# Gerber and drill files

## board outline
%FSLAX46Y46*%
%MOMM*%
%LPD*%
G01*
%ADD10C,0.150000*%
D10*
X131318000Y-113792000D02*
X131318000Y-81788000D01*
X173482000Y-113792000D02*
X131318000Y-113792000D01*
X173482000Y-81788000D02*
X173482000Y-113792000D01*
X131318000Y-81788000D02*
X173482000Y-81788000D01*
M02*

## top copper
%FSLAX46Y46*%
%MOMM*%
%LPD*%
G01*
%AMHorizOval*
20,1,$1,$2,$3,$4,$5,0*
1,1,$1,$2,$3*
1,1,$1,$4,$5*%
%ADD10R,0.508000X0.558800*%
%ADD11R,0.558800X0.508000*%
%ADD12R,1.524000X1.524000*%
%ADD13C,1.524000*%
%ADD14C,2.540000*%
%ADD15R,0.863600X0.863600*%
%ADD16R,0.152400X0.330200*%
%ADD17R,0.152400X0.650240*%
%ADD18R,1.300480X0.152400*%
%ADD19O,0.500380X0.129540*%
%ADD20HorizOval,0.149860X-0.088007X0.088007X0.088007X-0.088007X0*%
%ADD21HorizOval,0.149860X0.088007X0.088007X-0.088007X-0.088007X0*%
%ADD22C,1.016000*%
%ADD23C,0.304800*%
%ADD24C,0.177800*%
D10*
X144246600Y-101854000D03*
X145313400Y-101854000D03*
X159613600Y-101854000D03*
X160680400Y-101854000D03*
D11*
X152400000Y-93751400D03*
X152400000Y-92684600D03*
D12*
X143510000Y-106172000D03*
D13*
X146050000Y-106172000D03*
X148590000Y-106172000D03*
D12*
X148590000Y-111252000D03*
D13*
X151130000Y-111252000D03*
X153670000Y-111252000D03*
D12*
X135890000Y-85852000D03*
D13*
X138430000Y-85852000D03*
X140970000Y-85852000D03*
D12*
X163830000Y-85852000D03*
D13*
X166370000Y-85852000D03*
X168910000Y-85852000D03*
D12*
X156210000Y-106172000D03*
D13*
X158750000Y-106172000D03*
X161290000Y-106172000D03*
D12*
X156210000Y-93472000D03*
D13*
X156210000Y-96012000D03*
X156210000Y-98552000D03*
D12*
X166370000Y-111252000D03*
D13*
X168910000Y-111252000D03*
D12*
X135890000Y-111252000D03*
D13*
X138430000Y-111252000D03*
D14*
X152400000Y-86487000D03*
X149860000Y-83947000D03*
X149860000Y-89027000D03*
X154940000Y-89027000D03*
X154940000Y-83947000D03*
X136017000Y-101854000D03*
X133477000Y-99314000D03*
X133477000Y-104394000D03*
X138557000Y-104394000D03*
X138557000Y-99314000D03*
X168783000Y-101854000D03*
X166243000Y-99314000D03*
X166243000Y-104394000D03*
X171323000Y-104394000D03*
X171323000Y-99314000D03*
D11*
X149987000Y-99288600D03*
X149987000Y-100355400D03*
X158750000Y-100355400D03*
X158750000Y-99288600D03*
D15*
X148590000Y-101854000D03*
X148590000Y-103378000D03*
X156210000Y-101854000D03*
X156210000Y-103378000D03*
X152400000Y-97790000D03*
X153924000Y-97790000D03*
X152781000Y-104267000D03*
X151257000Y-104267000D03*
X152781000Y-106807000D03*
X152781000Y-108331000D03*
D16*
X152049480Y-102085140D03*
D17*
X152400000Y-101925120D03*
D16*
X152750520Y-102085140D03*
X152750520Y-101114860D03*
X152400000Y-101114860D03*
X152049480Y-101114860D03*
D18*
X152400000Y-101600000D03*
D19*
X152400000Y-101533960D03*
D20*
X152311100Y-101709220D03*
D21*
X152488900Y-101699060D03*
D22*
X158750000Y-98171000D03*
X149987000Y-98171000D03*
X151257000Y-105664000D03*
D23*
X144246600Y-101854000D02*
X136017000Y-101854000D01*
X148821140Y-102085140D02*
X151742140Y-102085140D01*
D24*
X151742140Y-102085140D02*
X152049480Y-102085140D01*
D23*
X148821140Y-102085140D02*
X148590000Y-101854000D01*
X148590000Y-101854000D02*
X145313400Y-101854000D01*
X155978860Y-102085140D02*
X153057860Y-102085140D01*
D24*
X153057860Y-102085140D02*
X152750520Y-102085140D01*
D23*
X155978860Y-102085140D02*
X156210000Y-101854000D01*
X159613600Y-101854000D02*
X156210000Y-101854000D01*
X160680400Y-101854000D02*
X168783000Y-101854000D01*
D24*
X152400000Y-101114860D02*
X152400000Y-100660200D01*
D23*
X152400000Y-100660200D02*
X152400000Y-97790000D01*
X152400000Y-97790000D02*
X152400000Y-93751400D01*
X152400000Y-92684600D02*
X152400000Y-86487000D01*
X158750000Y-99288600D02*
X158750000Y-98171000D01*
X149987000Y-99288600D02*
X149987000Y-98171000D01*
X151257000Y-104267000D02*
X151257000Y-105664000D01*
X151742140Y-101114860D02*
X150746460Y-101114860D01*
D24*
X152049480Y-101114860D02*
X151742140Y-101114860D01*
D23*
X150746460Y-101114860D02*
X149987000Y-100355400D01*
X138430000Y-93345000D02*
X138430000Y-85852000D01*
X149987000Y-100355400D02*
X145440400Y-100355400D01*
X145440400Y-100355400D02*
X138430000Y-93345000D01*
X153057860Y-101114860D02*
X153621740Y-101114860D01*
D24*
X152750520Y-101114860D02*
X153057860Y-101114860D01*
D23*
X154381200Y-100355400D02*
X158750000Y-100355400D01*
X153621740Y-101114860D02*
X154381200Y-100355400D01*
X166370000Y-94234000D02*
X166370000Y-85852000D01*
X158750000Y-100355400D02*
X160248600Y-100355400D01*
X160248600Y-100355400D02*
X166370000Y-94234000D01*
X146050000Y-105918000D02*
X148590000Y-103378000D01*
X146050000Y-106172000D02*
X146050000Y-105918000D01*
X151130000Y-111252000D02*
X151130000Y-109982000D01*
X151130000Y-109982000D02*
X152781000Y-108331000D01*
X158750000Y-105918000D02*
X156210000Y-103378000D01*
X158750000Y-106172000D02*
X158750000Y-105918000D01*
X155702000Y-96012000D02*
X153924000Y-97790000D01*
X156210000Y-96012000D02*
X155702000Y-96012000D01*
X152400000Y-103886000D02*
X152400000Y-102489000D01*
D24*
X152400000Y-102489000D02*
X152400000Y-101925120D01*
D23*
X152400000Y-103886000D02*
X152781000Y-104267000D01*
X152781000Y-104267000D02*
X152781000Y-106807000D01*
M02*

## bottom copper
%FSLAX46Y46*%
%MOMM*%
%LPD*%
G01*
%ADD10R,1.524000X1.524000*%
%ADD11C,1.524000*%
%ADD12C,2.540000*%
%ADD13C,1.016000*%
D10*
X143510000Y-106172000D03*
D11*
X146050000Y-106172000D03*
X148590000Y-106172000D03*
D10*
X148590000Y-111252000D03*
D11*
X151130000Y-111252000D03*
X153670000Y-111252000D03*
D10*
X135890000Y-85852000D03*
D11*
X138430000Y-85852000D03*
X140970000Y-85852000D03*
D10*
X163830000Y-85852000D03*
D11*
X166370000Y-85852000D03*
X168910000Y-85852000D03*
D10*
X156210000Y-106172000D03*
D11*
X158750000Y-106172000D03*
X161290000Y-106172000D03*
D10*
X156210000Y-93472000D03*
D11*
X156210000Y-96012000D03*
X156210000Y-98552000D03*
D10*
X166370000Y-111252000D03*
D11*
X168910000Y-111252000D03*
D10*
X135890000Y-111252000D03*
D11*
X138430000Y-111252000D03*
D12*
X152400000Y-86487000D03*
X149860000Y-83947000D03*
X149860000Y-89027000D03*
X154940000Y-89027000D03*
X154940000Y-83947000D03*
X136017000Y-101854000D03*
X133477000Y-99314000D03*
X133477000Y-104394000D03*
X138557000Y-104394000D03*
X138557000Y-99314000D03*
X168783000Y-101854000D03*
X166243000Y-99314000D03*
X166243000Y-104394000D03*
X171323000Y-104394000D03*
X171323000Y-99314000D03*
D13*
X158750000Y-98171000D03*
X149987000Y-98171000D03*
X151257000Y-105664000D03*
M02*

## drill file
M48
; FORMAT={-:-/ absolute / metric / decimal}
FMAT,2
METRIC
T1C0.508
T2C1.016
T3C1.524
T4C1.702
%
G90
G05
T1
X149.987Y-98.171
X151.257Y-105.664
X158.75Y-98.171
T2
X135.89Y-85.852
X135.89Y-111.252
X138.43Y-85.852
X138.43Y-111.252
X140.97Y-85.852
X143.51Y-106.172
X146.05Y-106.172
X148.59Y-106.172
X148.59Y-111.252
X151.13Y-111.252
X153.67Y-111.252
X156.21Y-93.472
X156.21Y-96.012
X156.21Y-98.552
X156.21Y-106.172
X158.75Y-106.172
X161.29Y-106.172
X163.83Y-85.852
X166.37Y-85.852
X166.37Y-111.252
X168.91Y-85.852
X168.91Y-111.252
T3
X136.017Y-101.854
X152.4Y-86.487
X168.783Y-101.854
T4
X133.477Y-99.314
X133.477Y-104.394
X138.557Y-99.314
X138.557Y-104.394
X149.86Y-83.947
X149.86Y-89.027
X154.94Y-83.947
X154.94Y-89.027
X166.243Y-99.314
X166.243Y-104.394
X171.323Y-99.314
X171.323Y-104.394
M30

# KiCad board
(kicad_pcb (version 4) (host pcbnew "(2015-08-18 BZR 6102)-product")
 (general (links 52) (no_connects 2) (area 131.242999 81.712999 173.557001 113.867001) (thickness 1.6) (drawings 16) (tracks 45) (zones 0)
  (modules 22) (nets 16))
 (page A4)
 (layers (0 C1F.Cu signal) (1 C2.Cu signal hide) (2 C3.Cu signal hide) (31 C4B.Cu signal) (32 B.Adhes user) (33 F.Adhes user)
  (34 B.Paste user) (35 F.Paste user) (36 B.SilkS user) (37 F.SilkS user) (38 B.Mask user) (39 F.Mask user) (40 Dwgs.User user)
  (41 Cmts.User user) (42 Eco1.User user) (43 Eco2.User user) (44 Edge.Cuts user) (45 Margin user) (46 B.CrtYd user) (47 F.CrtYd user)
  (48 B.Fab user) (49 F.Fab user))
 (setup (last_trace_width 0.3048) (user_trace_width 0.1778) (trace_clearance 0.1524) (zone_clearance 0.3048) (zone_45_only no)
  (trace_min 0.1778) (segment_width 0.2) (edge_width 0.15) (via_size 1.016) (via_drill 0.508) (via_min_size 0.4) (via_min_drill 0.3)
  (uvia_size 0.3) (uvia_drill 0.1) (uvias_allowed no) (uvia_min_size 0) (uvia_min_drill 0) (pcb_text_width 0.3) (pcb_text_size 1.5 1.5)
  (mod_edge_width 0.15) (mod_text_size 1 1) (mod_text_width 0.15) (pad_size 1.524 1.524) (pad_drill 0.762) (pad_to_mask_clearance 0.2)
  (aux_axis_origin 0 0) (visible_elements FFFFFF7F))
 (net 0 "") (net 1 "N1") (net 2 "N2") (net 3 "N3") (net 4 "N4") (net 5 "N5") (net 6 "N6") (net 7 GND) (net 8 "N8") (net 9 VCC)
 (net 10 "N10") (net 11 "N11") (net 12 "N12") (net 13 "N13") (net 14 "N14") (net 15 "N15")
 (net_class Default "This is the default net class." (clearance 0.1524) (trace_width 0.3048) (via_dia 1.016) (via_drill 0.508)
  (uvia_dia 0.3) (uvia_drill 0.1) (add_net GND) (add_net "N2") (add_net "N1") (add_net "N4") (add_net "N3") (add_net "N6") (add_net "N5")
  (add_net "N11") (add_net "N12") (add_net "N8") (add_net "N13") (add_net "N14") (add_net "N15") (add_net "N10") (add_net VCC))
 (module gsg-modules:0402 (layer C1F.Cu) (at 144.78 101.854 180) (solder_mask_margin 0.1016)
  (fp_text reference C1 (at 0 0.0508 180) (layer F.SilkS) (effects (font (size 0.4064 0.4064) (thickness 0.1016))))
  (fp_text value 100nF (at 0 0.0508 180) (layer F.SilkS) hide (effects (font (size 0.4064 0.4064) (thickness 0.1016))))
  (pad 2 smd rect (at 0.5334 0 180) (size 0.508 0.5588) (layers C1F.Cu F.Paste F.Mask) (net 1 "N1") (solder_mask_margin 0.1016))
  (pad 1 smd rect (at -0.5334 0 180) (size 0.508 0.5588) (layers C1F.Cu F.Paste F.Mask) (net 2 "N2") (solder_mask_margin 0.1016)))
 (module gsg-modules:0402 (layer C1F.Cu) (at 160.147 101.854 180) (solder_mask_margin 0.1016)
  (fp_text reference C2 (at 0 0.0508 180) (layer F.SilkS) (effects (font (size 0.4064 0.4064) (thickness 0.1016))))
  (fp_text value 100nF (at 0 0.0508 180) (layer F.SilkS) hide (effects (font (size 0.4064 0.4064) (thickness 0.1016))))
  (pad 2 smd rect (at 0.5334 0 180) (size 0.508 0.5588) (layers C1F.Cu F.Paste F.Mask) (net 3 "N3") (solder_mask_margin 0.1016))
  (pad 1 smd rect (at -0.5334 0 180) (size 0.508 0.5588) (layers C1F.Cu F.Paste F.Mask) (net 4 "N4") (solder_mask_margin 0.1016)))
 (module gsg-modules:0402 (layer C1F.Cu) (at 152.4 93.218 270) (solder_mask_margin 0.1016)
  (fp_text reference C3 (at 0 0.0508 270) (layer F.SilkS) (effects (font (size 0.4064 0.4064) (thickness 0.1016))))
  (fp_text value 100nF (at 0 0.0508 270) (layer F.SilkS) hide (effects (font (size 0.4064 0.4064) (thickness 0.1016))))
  (pad 2 smd rect (at 0.5334 0 270) (size 0.508 0.5588) (layers C1F.Cu F.Paste F.Mask) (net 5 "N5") (solder_mask_margin 0.1016))
  (pad 1 smd rect (at -0.5334 0 270) (size 0.508 0.5588) (layers C1F.Cu F.Paste F.Mask) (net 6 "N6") (solder_mask_margin 0.1016)))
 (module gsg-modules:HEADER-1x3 (layer C1F.Cu) (at 146.05 106.172)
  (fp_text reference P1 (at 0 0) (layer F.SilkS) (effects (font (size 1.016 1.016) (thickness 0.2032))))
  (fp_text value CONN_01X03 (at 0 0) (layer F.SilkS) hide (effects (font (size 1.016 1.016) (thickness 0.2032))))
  (pad 1 thru_hole rect (at -2.54 0) (size 1.524 1.524) (drill 1.016) (layers *.Cu *.Mask F.SilkS) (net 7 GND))
  (pad 2 thru_hole circle (at 0 0) (size 1.524 1.524) (drill 1.016) (layers *.Cu *.Mask F.SilkS) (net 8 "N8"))
  (pad 3 thru_hole circle (at 2.54 0) (size 1.524 1.524) (drill 1.016) (layers *.Cu *.Mask F.SilkS) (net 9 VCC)))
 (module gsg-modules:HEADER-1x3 (layer C1F.Cu) (at 151.13 111.252)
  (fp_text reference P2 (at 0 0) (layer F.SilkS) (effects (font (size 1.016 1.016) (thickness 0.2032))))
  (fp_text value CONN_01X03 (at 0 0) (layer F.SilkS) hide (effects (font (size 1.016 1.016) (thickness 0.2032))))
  (pad 1 thru_hole rect (at -2.54 0) (size 1.524 1.524) (drill 1.016) (layers *.Cu *.Mask F.SilkS) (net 7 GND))
  (pad 2 thru_hole circle (at 0 0) (size 1.524 1.524) (drill 1.016) (layers *.Cu *.Mask F.SilkS) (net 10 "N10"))
  (pad 3 thru_hole circle (at 2.54 0) (size 1.524 1.524) (drill 1.016) (layers *.Cu *.Mask F.SilkS) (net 9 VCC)))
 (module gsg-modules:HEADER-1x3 (layer C1F.Cu) (at 138.43 85.852)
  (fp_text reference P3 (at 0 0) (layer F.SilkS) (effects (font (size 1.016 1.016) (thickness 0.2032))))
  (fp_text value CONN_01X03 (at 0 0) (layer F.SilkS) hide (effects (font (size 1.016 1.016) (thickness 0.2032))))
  (pad 1 thru_hole rect (at -2.54 0) (size 1.524 1.524) (drill 1.016) (layers *.Cu *.Mask F.SilkS) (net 7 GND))
  (pad 2 thru_hole circle (at 0 0) (size 1.524 1.524) (drill 1.016) (layers *.Cu *.Mask F.SilkS) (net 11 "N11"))
  (pad 3 thru_hole circle (at 2.54 0) (size 1.524 1.524) (drill 1.016) (layers *.Cu *.Mask F.SilkS) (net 9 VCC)))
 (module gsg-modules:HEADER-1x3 (layer C1F.Cu) (at 166.37 85.852)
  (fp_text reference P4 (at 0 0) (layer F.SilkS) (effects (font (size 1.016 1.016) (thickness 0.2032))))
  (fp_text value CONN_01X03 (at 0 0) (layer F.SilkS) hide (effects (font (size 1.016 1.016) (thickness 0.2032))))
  (pad 1 thru_hole rect (at -2.54 0) (size 1.524 1.524) (drill 1.016) (layers *.Cu *.Mask F.SilkS) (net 7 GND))
  (pad 2 thru_hole circle (at 0 0) (size 1.524 1.524) (drill 1.016) (layers *.Cu *.Mask F.SilkS) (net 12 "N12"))
  (pad 3 thru_hole circle (at 2.54 0) (size 1.524 1.524) (drill 1.016) (layers *.Cu *.Mask F.SilkS) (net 9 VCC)))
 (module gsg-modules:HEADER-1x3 (layer C1F.Cu) (at 158.75 106.172)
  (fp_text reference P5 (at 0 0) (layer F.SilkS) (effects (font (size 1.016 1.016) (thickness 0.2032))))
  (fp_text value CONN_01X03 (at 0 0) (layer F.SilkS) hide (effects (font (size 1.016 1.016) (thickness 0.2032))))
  (pad 1 thru_hole rect (at -2.54 0) (size 1.524 1.524) (drill 1.016) (layers *.Cu *.Mask F.SilkS) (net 7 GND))
  (pad 2 thru_hole circle (at 0 0) (size 1.524 1.524) (drill 1.016) (layers *.Cu *.Mask F.SilkS) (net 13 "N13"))
  (pad 3 thru_hole circle (at 2.54 0) (size 1.524 1.524) (drill 1.016) (layers *.Cu *.Mask F.SilkS) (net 9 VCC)))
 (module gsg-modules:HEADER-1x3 (layer C1F.Cu) (at 156.21 96.012 270)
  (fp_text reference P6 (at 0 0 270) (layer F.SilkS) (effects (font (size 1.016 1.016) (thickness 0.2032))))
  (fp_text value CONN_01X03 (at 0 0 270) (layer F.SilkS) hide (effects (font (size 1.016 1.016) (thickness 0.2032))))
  (pad 1 thru_hole rect (at -2.54 0 270) (size 1.524 1.524) (drill 1.016) (layers *.Cu *.Mask F.SilkS) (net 7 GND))
  (pad 2 thru_hole circle (at 0 0 270) (size 1.524 1.524) (drill 1.016) (layers *.Cu *.Mask F.SilkS) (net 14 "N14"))
  (pad 3 thru_hole circle (at 2.54 0 270) (size 1.524 1.524) (drill 1.016) (layers *.Cu *.Mask F.SilkS) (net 9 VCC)))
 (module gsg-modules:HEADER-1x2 (layer C1F.Cu) (at 167.64 111.252)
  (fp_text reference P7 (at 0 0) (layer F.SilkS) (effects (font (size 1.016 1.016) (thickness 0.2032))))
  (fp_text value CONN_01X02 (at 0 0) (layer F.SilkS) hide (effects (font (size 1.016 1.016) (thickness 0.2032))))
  (pad 1 thru_hole rect (at -1.27 0) (size 1.524 1.524) (drill 1.016) (layers *.Cu *.Mask F.SilkS) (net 9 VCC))
  (pad 2 thru_hole circle (at 1.27 0) (size 1.524 1.524) (drill 1.016) (layers *.Cu *.Mask F.SilkS) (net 9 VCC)))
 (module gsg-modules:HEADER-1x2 (layer C1F.Cu) (at 137.16 111.252)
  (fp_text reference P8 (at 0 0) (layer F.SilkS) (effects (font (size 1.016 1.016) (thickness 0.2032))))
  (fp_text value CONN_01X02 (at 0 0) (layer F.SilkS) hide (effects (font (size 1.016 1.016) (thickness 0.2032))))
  (pad 1 thru_hole rect (at -1.27 0) (size 1.524 1.524) (drill 1.016) (layers *.Cu *.Mask F.SilkS) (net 7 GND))
  (pad 2 thru_hole circle (at 1.27 0) (size 1.524 1.524) (drill 1.016) (layers *.Cu *.Mask F.SilkS) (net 7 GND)))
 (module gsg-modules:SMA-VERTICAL (layer C1F.Cu) (at 152.4 86.487)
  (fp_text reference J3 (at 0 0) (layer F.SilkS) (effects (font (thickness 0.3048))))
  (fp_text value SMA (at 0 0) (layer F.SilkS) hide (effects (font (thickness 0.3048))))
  (pad 1 thru_hole circle (at 0 0) (size 2.54 2.54) (drill 1.524) (layers *.Cu *.Mask F.SilkS) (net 6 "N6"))
  (pad 2 thru_hole circle (at -2.54 -2.54) (size 2.54 2.54) (drill 1.7018) (layers *.Cu *.Mask F.SilkS) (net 7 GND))
  (pad 2 thru_hole circle (at -2.54 2.54) (size 2.54 2.54) (drill 1.7018) (layers *.Cu *.Mask F.SilkS) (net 7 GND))
  (pad 2 thru_hole circle (at 2.54 2.54) (size 2.54 2.54) (drill 1.7018) (layers *.Cu *.Mask F.SilkS) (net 7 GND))
  (pad 2 thru_hole circle (at 2.54 -2.54) (size 2.54 2.54) (drill 1.7018) (layers *.Cu *.Mask F.SilkS) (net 7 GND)))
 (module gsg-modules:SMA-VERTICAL (layer C1F.Cu) (at 136.017 101.854)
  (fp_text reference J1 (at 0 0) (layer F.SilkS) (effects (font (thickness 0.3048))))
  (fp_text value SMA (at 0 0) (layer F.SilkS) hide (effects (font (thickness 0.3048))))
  (pad 1 thru_hole circle (at 0 0) (size 2.54 2.54) (drill 1.524) (layers *.Cu *.Mask F.SilkS) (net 1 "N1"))
  (pad 2 thru_hole circle (at -2.54 -2.54) (size 2.54 2.54) (drill 1.7018) (layers *.Cu *.Mask F.SilkS) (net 7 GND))
  (pad 2 thru_hole circle (at -2.54 2.54) (size 2.54 2.54) (drill 1.7018) (layers *.Cu *.Mask F.SilkS) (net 7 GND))
  (pad 2 thru_hole circle (at 2.54 2.54) (size 2.54 2.54) (drill 1.7018) (layers *.Cu *.Mask F.SilkS) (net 7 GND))
  (pad 2 thru_hole circle (at 2.54 -2.54) (size 2.54 2.54) (drill 1.7018) (layers *.Cu *.Mask F.SilkS) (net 7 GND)))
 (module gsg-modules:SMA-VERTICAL (layer C1F.Cu) (at 168.783 101.854)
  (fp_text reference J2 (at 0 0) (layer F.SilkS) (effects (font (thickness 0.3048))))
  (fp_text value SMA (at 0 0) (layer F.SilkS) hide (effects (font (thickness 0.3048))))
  (pad 1 thru_hole circle (at 0 0) (size 2.54 2.54) (drill 1.524) (layers *.Cu *.Mask F.SilkS) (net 4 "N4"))
  (pad 2 thru_hole circle (at -2.54 -2.54) (size 2.54 2.54) (drill 1.7018) (layers *.Cu *.Mask F.SilkS) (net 7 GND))
  (pad 2 thru_hole circle (at -2.54 2.54) (size 2.54 2.54) (drill 1.7018) (layers *.Cu *.Mask F.SilkS) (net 7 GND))
  (pad 2 thru_hole circle (at 2.54 2.54) (size 2.54 2.54) (drill 1.7018) (layers *.Cu *.Mask F.SilkS) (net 7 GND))
  (pad 2 thru_hole circle (at 2.54 -2.54) (size 2.54 2.54) (drill 1.7018) (layers *.Cu *.Mask F.SilkS) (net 7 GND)))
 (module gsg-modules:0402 (layer C1F.Cu) (at 149.987 99.822 90) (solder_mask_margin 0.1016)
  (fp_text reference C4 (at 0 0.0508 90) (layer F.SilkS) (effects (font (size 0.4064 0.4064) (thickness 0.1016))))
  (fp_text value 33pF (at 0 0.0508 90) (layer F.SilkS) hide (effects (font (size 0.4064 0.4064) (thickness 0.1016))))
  (pad 2 smd rect (at 0.5334 0 90) (size 0.508 0.5588) (layers C1F.Cu F.Paste F.Mask) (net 7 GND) (solder_mask_margin 0.1016))
  (pad 1 smd rect (at -0.5334 0 90) (size 0.508 0.5588) (layers C1F.Cu F.Paste F.Mask) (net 11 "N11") (solder_mask_margin 0.1016)))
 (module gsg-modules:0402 (layer C1F.Cu) (at 158.75 99.822 270) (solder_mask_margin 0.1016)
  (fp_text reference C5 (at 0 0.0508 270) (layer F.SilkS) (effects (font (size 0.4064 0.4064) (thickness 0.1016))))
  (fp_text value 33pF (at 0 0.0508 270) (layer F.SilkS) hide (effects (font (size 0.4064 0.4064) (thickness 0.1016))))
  (pad 2 smd rect (at 0.5334 0 270) (size 0.508 0.5588) (layers C1F.Cu F.Paste F.Mask) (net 12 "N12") (solder_mask_margin 0.1016))
  (pad 1 smd rect (at -0.5334 0 270) (size 0.508 0.5588) (layers C1F.Cu F.Paste F.Mask) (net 7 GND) (solder_mask_margin 0.1016)))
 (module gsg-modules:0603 (layer C1F.Cu) (at 148.59 102.616 90) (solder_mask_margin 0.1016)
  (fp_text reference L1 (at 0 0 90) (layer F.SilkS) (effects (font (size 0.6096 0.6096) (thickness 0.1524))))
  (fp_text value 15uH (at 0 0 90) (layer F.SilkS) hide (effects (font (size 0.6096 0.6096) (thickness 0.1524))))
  (pad 2 smd rect (at 0.762 0 90) (size 0.8636 0.8636) (layers C1F.Cu F.Paste F.Mask) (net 2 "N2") (solder_mask_margin 0.1016)
   (clearance 0.1778))
  (pad 1 smd rect (at -0.762 0 90) (size 0.8636 0.8636) (layers C1F.Cu F.Paste F.Mask) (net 8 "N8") (solder_mask_margin 0.1016)
   (clearance 0.1778)))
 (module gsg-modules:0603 (layer C1F.Cu) (at 156.21 102.616 90) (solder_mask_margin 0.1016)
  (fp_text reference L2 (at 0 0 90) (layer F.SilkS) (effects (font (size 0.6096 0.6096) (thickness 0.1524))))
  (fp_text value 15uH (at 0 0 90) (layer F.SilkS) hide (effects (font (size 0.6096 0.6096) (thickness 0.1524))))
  (pad 2 smd rect (at 0.762 0 90) (size 0.8636 0.8636) (layers C1F.Cu F.Paste F.Mask) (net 3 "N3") (solder_mask_margin 0.1016)
   (clearance 0.1778))
  (pad 1 smd rect (at -0.762 0 90) (size 0.8636 0.8636) (layers C1F.Cu F.Paste F.Mask) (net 13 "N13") (solder_mask_margin 0.1016)
   (clearance 0.1778)))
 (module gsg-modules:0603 (layer C1F.Cu) (at 153.162 97.79 180) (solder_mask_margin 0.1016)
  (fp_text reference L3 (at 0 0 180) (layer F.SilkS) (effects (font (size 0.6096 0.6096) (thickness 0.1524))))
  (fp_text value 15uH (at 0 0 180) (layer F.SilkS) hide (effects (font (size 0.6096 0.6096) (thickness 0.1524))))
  (pad 2 smd rect (at 0.762 0 180) (size 0.8636 0.8636) (layers C1F.Cu F.Paste F.Mask) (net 5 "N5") (solder_mask_margin 0.1016)
   (clearance 0.1778))
  (pad 1 smd rect (at -0.762 0 180) (size 0.8636 0.8636) (layers C1F.Cu F.Paste F.Mask) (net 14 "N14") (solder_mask_margin 0.1016)
   (clearance 0.1778)))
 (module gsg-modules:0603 (layer C1F.Cu) (at 152.019 104.267) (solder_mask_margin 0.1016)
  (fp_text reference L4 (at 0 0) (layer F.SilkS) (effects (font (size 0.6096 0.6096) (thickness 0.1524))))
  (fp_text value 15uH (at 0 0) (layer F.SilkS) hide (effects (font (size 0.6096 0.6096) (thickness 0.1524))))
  (pad 2 smd rect (at 0.762 0) (size 0.8636 0.8636) (layers C1F.Cu F.Paste F.Mask) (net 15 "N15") (solder_mask_margin 0.1016)
   (clearance 0.1778))
  (pad 1 smd rect (at -0.762 0) (size 0.8636 0.8636) (layers C1F.Cu F.Paste F.Mask) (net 7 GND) (solder_mask_margin 0.1016)
   (clearance 0.1778)))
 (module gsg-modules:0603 (layer C1F.Cu) (at 152.781 107.569 90) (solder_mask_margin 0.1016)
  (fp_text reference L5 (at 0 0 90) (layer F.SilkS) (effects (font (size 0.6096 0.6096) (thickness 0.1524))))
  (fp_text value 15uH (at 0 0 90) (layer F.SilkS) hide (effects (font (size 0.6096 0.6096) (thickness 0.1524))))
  (pad 2 smd rect (at 0.762 0 90) (size 0.8636 0.8636) (layers C1F.Cu F.Paste F.Mask) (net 15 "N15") (solder_mask_margin 0.1016)
   (clearance 0.1778))
  (pad 1 smd rect (at -0.762 0 90) (size 0.8636 0.8636) (layers C1F.Cu F.Paste F.Mask) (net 10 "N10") (solder_mask_margin 0.1016)
   (clearance 0.1778)))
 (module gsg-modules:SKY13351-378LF (layer C1F.Cu) (at 152.4 101.6 90) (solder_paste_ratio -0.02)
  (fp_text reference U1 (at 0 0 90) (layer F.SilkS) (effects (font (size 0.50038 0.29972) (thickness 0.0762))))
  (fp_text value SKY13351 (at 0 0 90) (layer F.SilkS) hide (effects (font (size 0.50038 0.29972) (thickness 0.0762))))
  (pad 1 smd rect (at -0.48514 -0.35052 90) (size 0.3302 0.1524) (layers C1F.Cu F.Paste F.Mask) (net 2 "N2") (die_length -2147.483648))
  (pad 2 smd rect (at -0.32512 0 90) (size 0.65024 0.1524) (layers C1F.Cu F.Paste F.Mask) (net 15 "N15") (die_length -2147.483648))
  (pad 3 smd rect (at -0.48514 0.35052 90) (size 0.3302 0.1524) (layers C1F.Cu F.Paste F.Mask) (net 3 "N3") (die_length -2147.483648))
  (pad 4 smd rect (at 0.48514 0.35052 90) (size 0.3302 0.1524) (layers C1F.Cu F.Paste F.Mask) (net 12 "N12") (die_length 0.0508))
  (pad 5 smd rect (at 0.48514 0 90) (size 0.3302 0.1524) (layers C1F.Cu F.Paste F.Mask) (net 5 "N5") (die_length 10.53846))
  (pad 6 smd rect (at 0.48514 -0.35052 90) (size 0.3302 0.1524) (layers C1F.Cu F.Paste F.Mask) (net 11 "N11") (die_length -2147.483648))
  (pad 2 smd rect (at 0 0 90) (size 0.1524 1.30048) (layers C1F.Cu F.Paste F.Mask) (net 15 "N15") (die_length -2147.483648))
  (pad 2 smd oval (at 0.06604 0 90) (size 0.12954 0.50038) (layers C1F.Cu F.Paste F.Mask) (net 15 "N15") (die_length -2147.483648))
  (pad 2 smd oval (at -0.10922 -0.0889 45) (size 0.14986 0.39878) (layers C1F.Cu F.Paste F.Mask) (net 15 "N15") (die_length -2147.483648))
  (pad 2 smd oval (at -0.09906 0.0889 135) (size 0.14986 0.39878) (layers C1F.Cu F.Paste F.Mask) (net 15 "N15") (die_length -2147.483648)))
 (gr_line (start 131.318 113.792) (end 131.318 81.788) (angle 90) (layer Edge.Cuts) (width 0.15))
 (gr_line (start 173.482 113.792) (end 131.318 113.792) (angle 90) (layer Edge.Cuts) (width 0.15))
 (gr_line (start 173.482 81.788) (end 173.482 113.792) (angle 90) (layer Edge.Cuts) (width 0.15))
 (gr_line (start 131.318 81.788) (end 173.482 81.788) (angle 90) (layer Edge.Cuts) (width 0.15))
 (segment (start 144.2466 101.854) (end 136.017 101.854) (width 0.3048) (layer C1F.Cu) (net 1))
 (segment (start 148.82114 102.08514) (end 151.74214 102.08514) (width 0.3048) (layer C1F.Cu) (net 2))
 (segment (start 151.74214 102.08514) (end 152.04948 102.08514) (width 0.1778) (layer C1F.Cu) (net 2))
 (segment (start 148.82114 102.08514) (end 148.59 101.854) (width 0.3048) (layer C1F.Cu) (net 2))
 (segment (start 148.59 101.854) (end 145.3134 101.854) (width 0.3048) (layer C1F.Cu) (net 2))
 (segment (start 155.97886 102.08514) (end 153.05786 102.08514) (width 0.3048) (layer C1F.Cu) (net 3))
 (segment (start 153.05786 102.08514) (end 152.75052 102.08514) (width 0.1778) (layer C1F.Cu) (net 3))
 (segment (start 155.97886 102.08514) (end 156.21 101.854) (width 0.3048) (layer C1F.Cu) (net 3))
 (segment (start 159.6136 101.854) (end 156.21 101.854) (width 0.3048) (layer C1F.Cu) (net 3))
 (segment (start 160.6804 101.854) (end 168.783 101.854) (width 0.3048) (layer C1F.Cu) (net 4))
 (segment (start 152.4 101.11486) (end 152.4 100.6602) (width 0.1778) (layer C1F.Cu) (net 5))
 (segment (start 152.4 100.6602) (end 152.4 97.79) (width 0.3048) (layer C1F.Cu) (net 5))
 (segment (start 152.4 97.79) (end 152.4 93.7514) (width 0.3048) (layer C1F.Cu) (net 5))
 (segment (start 152.4 92.6846) (end 152.4 86.487) (width 0.3048) (layer C1F.Cu) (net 6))
 (segment (start 158.75 99.2886) (end 158.75 98.171) (width 0.3048) (layer C1F.Cu) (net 7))
 (via (at 158.75 98.171) (size 1.016) (drill 0.508) (layers C1F.Cu C4B.Cu) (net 7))
 (segment (start 149.987 99.2886) (end 149.987 98.171) (width 0.3048) (layer C1F.Cu) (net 7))
 (via (at 149.987 98.171) (size 1.016) (drill 0.508) (layers C1F.Cu C4B.Cu) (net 7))
 (segment (start 151.257 104.267) (end 151.257 105.664) (width 0.3048) (layer C1F.Cu) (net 7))
 (via (at 151.257 105.664) (size 1.016) (drill 0.508) (layers C1F.Cu C4B.Cu) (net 7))
 (segment (start 151.74214 101.11486) (end 150.74646 101.11486) (width 0.3048) (layer C1F.Cu) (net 11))
 (segment (start 152.04948 101.11486) (end 151.74214 101.11486) (width 0.1778) (layer C1F.Cu) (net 11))
 (segment (start 150.74646 101.11486) (end 149.987 100.3554) (width 0.3048) (layer C1F.Cu) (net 11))
 (segment (start 138.43 93.345) (end 138.43 85.852) (width 0.3048) (layer C1F.Cu) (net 11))
 (segment (start 149.987 100.3554) (end 145.4404 100.3554) (width 0.3048) (layer C1F.Cu) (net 11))
 (segment (start 145.4404 100.3554) (end 138.43 93.345) (width 0.3048) (layer C1F.Cu) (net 11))
 (segment (start 153.05786 101.11486) (end 153.62174 101.11486) (width 0.3048) (layer C1F.Cu) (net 12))
 (segment (start 152.75052 101.11486) (end 153.05786 101.11486) (width 0.1778) (layer C1F.Cu) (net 12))
 (segment (start 154.3812 100.3554) (end 158.75 100.3554) (width 0.3048) (layer C1F.Cu) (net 12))
 (segment (start 153.62174 101.11486) (end 154.3812 100.3554) (width 0.3048) (layer C1F.Cu) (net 12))
 (segment (start 166.37 94.234) (end 166.37 85.852) (width 0.3048) (layer C1F.Cu) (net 12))
 (segment (start 158.75 100.3554) (end 160.2486 100.3554) (width 0.3048) (layer C1F.Cu) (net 12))
 (segment (start 160.2486 100.3554) (end 166.37 94.234) (width 0.3048) (layer C1F.Cu) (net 12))
 (segment (start 146.05 105.918) (end 148.59 103.378) (width 0.3048) (layer C1F.Cu) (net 8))
 (segment (start 146.05 106.172) (end 146.05 105.918) (width 0.3048) (layer C1F.Cu) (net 8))
 (segment (start 151.13 111.252) (end 151.13 109.982) (width 0.3048) (layer C1F.Cu) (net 10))
 (segment (start 151.13 109.982) (end 152.781 108.331) (width 0.3048) (layer C1F.Cu) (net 10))
 (segment (start 158.75 105.918) (end 156.21 103.378) (width 0.3048) (layer C1F.Cu) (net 13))
 (segment (start 158.75 106.172) (end 158.75 105.918) (width 0.3048) (layer C1F.Cu) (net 13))
 (segment (start 155.702 96.012) (end 153.924 97.79) (width 0.3048) (layer C1F.Cu) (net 14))
 (segment (start 156.21 96.012) (end 155.702 96.012) (width 0.3048) (layer C1F.Cu) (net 14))
 (segment (start 152.4 103.886) (end 152.4 102.489) (width 0.3048) (layer C1F.Cu) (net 15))
 (segment (start 152.4 102.489) (end 152.4 101.92512) (width 0.1778) (layer C1F.Cu) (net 15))
 (segment (start 152.4 103.886) (end 152.781 104.267) (width 0.3048) (layer C1F.Cu) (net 15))
 (segment (start 152.781 104.267) (end 152.781 106.807) (width 0.3048) (layer C1F.Cu) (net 15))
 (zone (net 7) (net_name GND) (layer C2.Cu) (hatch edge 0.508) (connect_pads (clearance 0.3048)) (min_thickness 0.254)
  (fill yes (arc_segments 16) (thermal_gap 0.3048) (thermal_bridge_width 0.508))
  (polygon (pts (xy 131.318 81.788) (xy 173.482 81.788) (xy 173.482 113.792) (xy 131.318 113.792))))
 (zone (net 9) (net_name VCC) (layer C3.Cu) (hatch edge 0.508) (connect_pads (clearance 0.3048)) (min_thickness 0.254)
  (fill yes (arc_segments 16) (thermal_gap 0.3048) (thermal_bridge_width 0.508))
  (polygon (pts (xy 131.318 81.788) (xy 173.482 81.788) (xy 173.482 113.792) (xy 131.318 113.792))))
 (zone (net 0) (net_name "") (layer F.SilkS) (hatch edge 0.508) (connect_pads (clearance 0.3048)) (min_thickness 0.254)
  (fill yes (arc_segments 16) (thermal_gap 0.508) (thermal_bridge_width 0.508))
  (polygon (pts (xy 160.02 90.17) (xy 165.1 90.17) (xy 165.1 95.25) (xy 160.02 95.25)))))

